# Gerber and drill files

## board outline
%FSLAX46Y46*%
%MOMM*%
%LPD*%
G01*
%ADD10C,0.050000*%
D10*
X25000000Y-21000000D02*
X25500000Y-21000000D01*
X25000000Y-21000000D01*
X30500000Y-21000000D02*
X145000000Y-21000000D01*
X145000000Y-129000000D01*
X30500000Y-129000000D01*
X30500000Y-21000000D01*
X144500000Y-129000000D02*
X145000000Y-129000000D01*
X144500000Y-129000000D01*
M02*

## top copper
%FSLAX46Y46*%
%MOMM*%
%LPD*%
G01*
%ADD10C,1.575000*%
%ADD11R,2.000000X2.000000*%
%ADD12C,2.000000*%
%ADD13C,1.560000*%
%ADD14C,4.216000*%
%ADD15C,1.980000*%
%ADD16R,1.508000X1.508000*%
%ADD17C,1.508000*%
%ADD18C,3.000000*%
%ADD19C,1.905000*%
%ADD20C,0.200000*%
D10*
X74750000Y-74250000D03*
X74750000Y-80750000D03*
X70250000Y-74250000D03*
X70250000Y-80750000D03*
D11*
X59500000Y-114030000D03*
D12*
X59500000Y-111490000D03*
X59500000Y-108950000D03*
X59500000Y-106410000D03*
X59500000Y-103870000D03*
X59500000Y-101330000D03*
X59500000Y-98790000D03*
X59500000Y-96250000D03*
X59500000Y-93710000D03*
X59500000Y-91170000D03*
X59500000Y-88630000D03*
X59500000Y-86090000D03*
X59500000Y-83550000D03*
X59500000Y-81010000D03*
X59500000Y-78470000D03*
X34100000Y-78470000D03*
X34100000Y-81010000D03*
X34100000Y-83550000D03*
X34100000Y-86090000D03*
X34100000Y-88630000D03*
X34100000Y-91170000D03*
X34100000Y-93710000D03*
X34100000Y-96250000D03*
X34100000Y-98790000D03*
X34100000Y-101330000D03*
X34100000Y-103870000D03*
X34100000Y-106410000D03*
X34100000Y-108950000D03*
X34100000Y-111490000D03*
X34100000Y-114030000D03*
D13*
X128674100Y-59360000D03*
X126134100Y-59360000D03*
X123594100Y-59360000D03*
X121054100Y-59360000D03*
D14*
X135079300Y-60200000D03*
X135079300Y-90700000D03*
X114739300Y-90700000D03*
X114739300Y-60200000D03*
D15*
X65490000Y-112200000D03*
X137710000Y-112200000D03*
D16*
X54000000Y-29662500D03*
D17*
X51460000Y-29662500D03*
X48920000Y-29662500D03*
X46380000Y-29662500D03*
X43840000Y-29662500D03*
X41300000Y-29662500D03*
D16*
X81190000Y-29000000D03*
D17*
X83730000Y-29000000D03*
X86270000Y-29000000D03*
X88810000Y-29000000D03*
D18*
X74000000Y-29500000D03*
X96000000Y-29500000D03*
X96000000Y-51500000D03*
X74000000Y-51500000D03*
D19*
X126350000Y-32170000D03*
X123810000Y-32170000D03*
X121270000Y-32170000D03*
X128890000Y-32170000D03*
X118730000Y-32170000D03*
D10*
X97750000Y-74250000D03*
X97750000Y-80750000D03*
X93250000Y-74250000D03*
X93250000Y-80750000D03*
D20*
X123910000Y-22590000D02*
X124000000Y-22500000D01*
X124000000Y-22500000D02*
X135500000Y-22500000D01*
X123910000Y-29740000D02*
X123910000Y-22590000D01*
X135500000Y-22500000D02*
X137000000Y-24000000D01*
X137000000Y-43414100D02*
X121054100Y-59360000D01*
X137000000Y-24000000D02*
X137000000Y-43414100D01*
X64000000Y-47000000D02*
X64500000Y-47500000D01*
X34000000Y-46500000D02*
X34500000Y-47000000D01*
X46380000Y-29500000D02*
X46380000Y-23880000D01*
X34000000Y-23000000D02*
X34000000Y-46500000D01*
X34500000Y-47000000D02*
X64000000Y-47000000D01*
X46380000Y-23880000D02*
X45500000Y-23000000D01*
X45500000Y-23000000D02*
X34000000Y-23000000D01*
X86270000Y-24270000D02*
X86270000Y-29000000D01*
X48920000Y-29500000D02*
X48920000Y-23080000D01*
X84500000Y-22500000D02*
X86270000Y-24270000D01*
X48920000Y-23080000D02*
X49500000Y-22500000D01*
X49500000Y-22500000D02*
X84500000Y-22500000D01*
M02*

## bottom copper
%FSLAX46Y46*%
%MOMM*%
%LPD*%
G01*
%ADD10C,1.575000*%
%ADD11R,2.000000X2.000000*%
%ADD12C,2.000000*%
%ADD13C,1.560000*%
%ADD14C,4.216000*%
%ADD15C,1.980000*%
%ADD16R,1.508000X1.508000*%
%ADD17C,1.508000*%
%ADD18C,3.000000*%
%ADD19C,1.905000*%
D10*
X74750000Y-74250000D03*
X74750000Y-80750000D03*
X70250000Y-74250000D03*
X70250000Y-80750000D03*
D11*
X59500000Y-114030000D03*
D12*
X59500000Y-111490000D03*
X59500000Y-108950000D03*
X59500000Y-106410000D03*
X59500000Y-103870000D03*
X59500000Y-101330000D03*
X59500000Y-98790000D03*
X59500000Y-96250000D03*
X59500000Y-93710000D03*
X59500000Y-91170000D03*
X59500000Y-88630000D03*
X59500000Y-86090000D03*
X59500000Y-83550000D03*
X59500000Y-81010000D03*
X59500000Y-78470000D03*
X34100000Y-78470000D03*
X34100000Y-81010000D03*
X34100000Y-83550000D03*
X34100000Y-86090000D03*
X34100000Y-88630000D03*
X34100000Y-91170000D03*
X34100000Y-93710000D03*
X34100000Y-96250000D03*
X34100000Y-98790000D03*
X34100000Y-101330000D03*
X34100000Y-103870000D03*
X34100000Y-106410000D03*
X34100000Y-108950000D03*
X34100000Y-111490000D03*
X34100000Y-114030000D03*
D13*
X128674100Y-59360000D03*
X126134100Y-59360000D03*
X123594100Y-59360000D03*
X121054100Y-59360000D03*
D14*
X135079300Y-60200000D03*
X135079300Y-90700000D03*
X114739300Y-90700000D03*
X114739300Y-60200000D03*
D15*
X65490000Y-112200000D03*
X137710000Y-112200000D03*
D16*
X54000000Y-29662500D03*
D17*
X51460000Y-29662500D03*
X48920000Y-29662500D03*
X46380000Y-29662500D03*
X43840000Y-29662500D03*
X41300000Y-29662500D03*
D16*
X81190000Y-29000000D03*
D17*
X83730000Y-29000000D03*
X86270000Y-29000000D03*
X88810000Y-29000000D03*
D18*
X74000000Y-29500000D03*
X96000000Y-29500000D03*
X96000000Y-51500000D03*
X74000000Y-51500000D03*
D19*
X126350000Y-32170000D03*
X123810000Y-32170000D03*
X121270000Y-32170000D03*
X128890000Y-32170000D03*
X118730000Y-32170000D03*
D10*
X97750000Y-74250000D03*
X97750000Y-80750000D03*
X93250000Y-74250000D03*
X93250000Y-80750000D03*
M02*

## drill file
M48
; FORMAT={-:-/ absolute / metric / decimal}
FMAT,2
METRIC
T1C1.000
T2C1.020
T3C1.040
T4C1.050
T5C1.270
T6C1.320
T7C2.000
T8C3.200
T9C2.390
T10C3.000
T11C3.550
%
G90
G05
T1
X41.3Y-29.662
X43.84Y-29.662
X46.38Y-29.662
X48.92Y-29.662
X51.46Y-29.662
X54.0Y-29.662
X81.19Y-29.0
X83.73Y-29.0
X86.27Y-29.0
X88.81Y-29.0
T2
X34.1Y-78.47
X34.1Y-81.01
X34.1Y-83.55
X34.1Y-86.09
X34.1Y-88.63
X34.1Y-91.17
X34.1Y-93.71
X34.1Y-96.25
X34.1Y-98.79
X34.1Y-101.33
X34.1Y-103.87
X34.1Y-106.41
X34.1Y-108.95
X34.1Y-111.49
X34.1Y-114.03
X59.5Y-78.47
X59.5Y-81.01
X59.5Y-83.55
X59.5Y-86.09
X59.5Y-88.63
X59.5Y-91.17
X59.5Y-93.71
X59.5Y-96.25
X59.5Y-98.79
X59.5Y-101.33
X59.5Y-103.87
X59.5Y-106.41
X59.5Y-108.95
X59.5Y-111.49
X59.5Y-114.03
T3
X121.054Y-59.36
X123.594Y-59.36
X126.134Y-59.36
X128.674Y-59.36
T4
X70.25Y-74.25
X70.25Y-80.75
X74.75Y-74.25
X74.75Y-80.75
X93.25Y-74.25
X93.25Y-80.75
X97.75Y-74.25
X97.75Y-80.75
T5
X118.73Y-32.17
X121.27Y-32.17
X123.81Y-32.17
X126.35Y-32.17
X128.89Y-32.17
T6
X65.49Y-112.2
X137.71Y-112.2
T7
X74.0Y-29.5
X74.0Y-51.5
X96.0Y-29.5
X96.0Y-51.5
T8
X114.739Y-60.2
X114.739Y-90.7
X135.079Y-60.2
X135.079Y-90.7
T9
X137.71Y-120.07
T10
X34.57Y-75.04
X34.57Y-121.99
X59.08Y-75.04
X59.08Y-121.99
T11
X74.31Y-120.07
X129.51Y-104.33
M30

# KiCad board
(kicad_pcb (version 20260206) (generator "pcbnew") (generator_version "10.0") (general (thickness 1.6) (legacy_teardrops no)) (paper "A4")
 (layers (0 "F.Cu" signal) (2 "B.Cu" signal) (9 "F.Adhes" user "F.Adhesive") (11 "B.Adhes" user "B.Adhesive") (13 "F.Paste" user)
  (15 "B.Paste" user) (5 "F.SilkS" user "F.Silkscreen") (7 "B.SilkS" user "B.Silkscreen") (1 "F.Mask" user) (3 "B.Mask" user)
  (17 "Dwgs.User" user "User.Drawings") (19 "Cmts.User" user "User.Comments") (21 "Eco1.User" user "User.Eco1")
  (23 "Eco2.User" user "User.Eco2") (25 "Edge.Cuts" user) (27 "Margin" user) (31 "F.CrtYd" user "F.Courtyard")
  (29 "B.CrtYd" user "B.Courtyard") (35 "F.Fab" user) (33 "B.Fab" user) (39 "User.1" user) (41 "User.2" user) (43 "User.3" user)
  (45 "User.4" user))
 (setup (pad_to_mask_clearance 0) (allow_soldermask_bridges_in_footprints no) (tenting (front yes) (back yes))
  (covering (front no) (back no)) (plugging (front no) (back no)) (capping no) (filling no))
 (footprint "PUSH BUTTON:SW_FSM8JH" (layer "F.Cu") (at 72.5 77.5)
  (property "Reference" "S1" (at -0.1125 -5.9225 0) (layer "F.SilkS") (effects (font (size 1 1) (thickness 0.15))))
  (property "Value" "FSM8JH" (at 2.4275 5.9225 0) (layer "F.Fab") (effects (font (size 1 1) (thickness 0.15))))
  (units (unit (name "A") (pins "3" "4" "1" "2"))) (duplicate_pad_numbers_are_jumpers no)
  (pad "1" thru_hole circle (at 2.25 -3.25) (size 1.575 1.575) (drill 1.05) (layers "*.Cu" "*.Mask") (remove_unused_layers no)
   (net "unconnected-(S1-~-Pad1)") (solder_mask_margin 0.102))
  (pad "2" thru_hole circle (at 2.25 3.25) (size 1.575 1.575) (drill 1.05) (layers "*.Cu" "*.Mask") (remove_unused_layers no)
   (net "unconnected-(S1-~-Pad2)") (solder_mask_margin 0.102))
  (pad "3" thru_hole circle (at -2.25 -3.25) (size 1.575 1.575) (drill 1.05) (layers "*.Cu" "*.Mask") (remove_unused_layers no)
   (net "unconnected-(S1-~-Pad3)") (solder_mask_margin 0.102))
  (pad "4" thru_hole circle (at -2.25 3.25) (size 1.575 1.575) (drill 1.05) (layers "*.Cu" "*.Mask") (remove_unused_layers no)
   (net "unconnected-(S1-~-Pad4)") (solder_mask_margin 0.102)))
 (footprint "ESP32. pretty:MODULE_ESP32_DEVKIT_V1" (layer "F.Cu") (at 46.8 98.515 180)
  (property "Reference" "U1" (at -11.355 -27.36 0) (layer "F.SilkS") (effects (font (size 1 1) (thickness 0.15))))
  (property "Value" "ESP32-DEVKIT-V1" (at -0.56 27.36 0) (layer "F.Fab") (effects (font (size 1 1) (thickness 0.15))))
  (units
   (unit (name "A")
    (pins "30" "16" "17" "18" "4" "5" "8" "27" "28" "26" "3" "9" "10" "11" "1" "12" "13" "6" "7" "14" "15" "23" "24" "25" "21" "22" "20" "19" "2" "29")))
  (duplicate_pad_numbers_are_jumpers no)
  (pad "" np_thru_hole circle (at -12.28 -23.475 180) (size 3 3) (drill 3) (layers "*.Cu" "*.Mask"))
  (pad "" np_thru_hole circle (at -12.28 23.475 180) (size 3 3) (drill 3) (layers "*.Cu" "*.Mask"))
  (pad "" np_thru_hole circle (at 12.23 -23.475 180) (size 3 3) (drill 3) (layers "*.Cu" "*.Mask"))
  (pad "" np_thru_hole circle (at 12.23 23.475 180) (size 3 3) (drill 3) (layers "*.Cu" "*.Mask"))
  (pad "1" thru_hole rect (at -12.7 -15.515 180) (size 2 2) (drill 1.02) (layers "*.Cu" "*.Mask") (remove_unused_layers no)
   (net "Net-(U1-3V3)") (solder_mask_margin 0.102))
  (pad "2" thru_hole circle (at -12.7 -12.975 180) (size 2 2) (drill 1.02) (layers "*.Cu" "*.Mask") (remove_unused_layers no)
   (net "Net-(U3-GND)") (solder_mask_margin 0.102))
  (pad "3" thru_hole circle (at -12.7 -10.435 180) (size 2 2) (drill 1.02) (layers "*.Cu" "*.Mask") (remove_unused_layers no)
   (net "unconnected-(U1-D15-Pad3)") (solder_mask_margin 0.102))
  (pad "4" thru_hole circle (at -12.7 -7.895 180) (size 2 2) (drill 1.02) (layers "*.Cu" "*.Mask") (remove_unused_layers no)
   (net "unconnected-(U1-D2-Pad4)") (solder_mask_margin 0.102))
  (pad "5" thru_hole circle (at -12.7 -5.355 180) (size 2 2) (drill 1.02) (layers "*.Cu" "*.Mask") (remove_unused_layers no)
   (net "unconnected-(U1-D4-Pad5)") (solder_mask_margin 0.102))
  (pad "6" thru_hole circle (at -12.7 -2.815 180) (size 2 2) (drill 1.02) (layers "*.Cu" "*.Mask") (remove_unused_layers no)
   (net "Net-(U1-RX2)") (solder_mask_margin 0.102))
  (pad "7" thru_hole circle (at -12.7 -0.275 180) (size 2 2) (drill 1.02) (layers "*.Cu" "*.Mask") (remove_unused_layers no)
   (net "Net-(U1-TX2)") (solder_mask_margin 0.102))
  (pad "8" thru_hole circle (at -12.7 2.265 180) (size 2 2) (drill 1.02) (layers "*.Cu" "*.Mask") (remove_unused_layers no)
   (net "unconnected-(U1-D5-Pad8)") (solder_mask_margin 0.102))
  (pad "9" thru_hole circle (at -12.7 4.805 180) (size 2 2) (drill 1.02) (layers "*.Cu" "*.Mask") (remove_unused_layers no)
   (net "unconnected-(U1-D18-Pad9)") (solder_mask_margin 0.102))
  (pad "10" thru_hole circle (at -12.7 7.345 180) (size 2 2) (drill 1.02) (layers "*.Cu" "*.Mask") (remove_unused_layers no)
   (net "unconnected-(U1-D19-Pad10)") (solder_mask_margin 0.102))
  (pad "11" thru_hole circle (at -12.7 9.885 180) (size 2 2) (drill 1.02) (layers "*.Cu" "*.Mask") (remove_unused_layers no)
   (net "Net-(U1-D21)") (solder_mask_margin 0.102))
  (pad "12" thru_hole circle (at -12.7 12.425 180) (size 2 2) (drill 1.02) (layers "*.Cu" "*.Mask") (remove_unused_layers no)
   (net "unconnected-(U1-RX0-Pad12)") (solder_mask_margin 0.102))
  (pad "13" thru_hole circle (at -12.7 14.965 180) (size 2 2) (drill 1.02) (layers "*.Cu" "*.Mask") (remove_unused_layers no)
   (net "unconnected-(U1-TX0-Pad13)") (solder_mask_margin 0.102))
  (pad "14" thru_hole circle (at -12.7 17.505 180) (size 2 2) (drill 1.02) (layers "*.Cu" "*.Mask") (remove_unused_layers no)
   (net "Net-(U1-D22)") (solder_mask_margin 0.102))
  (pad "15" thru_hole circle (at -12.7 20.045 180) (size 2 2) (drill 1.02) (layers "*.Cu" "*.Mask") (remove_unused_layers no)
   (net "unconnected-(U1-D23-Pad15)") (solder_mask_margin 0.102))
  (pad "16" thru_hole circle (at 12.7 20.045 180) (size 2 2) (drill 1.02) (layers "*.Cu" "*.Mask") (remove_unused_layers no)
   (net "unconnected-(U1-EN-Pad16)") (solder_mask_margin 0.102))
  (pad "17" thru_hole circle (at 12.7 17.505 180) (size 2 2) (drill 1.02) (layers "*.Cu" "*.Mask") (remove_unused_layers no)
   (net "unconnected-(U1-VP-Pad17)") (solder_mask_margin 0.102))
  (pad "18" thru_hole circle (at 12.7 14.965 180) (size 2 2) (drill 1.02) (layers "*.Cu" "*.Mask") (remove_unused_layers no)
   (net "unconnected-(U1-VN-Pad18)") (solder_mask_margin 0.102))
  (pad "19" thru_hole circle (at 12.7 12.425 180) (size 2 2) (drill 1.02) (layers "*.Cu" "*.Mask") (remove_unused_layers no)
   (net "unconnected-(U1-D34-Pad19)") (solder_mask_margin 0.102))
  (pad "20" thru_hole circle (at 12.7 9.885 180) (size 2 2) (drill 1.02) (layers "*.Cu" "*.Mask") (remove_unused_layers no)
   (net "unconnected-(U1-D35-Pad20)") (solder_mask_margin 0.102))
  (pad "21" thru_hole circle (at 12.7 7.345 180) (size 2 2) (drill 1.02) (layers "*.Cu" "*.Mask") (remove_unused_layers no)
   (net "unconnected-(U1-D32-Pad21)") (solder_mask_margin 0.102))
  (pad "22" thru_hole circle (at 12.7 4.805 180) (size 2 2) (drill 1.02) (layers "*.Cu" "*.Mask") (remove_unused_layers no)
   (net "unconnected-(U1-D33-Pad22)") (solder_mask_margin 0.102))
  (pad "23" thru_hole circle (at 12.7 2.265 180) (size 2 2) (drill 1.02) (layers "*.Cu" "*.Mask") (remove_unused_layers no)
   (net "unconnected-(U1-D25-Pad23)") (solder_mask_margin 0.102))
  (pad "24" thru_hole circle (at 12.7 -0.275 180) (size 2 2) (drill 1.02) (layers "*.Cu" "*.Mask") (remove_unused_layers no)
   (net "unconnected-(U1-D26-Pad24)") (solder_mask_margin 0.102))
  (pad "25" thru_hole circle (at 12.7 -2.815 180) (size 2 2) (drill 1.02) (layers "*.Cu" "*.Mask") (remove_unused_layers no)
   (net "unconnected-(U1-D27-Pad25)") (solder_mask_margin 0.102))
  (pad "26" thru_hole circle (at 12.7 -5.355 180) (size 2 2) (drill 1.02) (layers "*.Cu" "*.Mask") (remove_unused_layers no)
   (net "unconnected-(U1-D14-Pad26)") (solder_mask_margin 0.102))
  (pad "27" thru_hole circle (at 12.7 -7.895 180) (size 2 2) (drill 1.02) (layers "*.Cu" "*.Mask") (remove_unused_layers no)
   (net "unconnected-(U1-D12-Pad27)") (solder_mask_margin 0.102))
  (pad "28" thru_hole circle (at 12.7 -10.435 180) (size 2 2) (drill 1.02) (layers "*.Cu" "*.Mask") (remove_unused_layers no)
   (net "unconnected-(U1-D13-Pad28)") (solder_mask_margin 0.102))
  (pad "29" thru_hole circle (at 12.7 -12.975 180) (size 2 2) (drill 1.02) (layers "*.Cu" "*.Mask") (remove_unused_layers no)
   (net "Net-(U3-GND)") (solder_mask_margin 0.102))
  (pad "30" thru_hole circle (at 12.7 -15.515 180) (size 2 2) (drill 1.02) (layers "*.Cu" "*.Mask") (remove_unused_layers no)
   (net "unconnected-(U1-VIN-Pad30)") (solder_mask_margin 0.102)))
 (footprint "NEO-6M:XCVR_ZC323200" (layer "F.Cu") (at 124.5 75.5 180)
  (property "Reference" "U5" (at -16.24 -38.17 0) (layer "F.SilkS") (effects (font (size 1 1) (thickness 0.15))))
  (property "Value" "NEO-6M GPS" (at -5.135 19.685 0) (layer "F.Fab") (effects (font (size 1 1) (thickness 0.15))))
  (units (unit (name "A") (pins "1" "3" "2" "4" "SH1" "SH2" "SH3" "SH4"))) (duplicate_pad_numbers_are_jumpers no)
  (pad "1" thru_hole circle (at -4.1741 16.14 180) (size 1.56 1.56) (drill 1.04) (layers "*.Cu" "*.Mask") (remove_unused_layers no)
   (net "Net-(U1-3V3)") (solder_mask_margin 0.102))
  (pad "2" thru_hole circle (at -1.6341 16.14 180) (size 1.56 1.56) (drill 1.04) (layers "*.Cu" "*.Mask") (remove_unused_layers no)
   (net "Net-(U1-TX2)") (solder_mask_margin 0.102))
  (pad "3" thru_hole circle (at 0.9059 16.14 180) (size 1.56 1.56) (drill 1.04) (layers "*.Cu" "*.Mask") (remove_unused_layers no)
   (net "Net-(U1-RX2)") (solder_mask_margin 0.102))
  (pad "4" thru_hole circle (at 3.4459 16.14 180) (size 1.56 1.56) (drill 1.04) (layers "*.Cu" "*.Mask") (remove_unused_layers no)
   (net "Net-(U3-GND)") (solder_mask_margin 0.102))
  (pad "SH1" thru_hole circle (at -10.5793 15.3 180) (size 4.216 4.216) (drill 3.2) (layers "*.Cu" "*.Mask") (remove_unused_layers no)
   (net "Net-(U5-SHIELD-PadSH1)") (solder_mask_margin 0.102))
  (pad "SH2" thru_hole circle (at -10.5793 -15.2 180) (size 4.216 4.216) (drill 3.2) (layers "*.Cu" "*.Mask") (remove_unused_layers no)
   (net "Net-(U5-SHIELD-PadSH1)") (solder_mask_margin 0.102))
  (pad "SH3" thru_hole circle (at 9.7607 -15.2 180) (size 4.216 4.216) (drill 3.2) (layers "*.Cu" "*.Mask") (remove_unused_layers no)
   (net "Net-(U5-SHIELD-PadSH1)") (solder_mask_margin 0.102))
  (pad "SH4" thru_hole circle (at 9.7607 15.3 180) (size 4.216 4.216) (drill 3.2) (layers "*.Cu" "*.Mask") (remove_unused_layers no)
   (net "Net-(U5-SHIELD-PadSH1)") (solder_mask_margin 0.102)))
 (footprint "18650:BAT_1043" (layer "F.Cu") (at 101.6 112.2)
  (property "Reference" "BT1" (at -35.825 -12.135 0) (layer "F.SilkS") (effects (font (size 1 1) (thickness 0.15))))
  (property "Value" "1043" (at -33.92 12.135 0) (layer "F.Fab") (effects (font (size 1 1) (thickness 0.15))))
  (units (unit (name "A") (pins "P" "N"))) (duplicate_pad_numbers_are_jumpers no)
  (pad "" np_thru_hole circle (at -27.29 7.87) (size 3.55 3.55) (drill 3.55) (layers "*.Cu" "*.Mask"))
  (pad "" np_thru_hole circle (at 27.91 -7.87) (size 3.55 3.55) (drill 3.55) (layers "*.Cu" "*.Mask"))
  (pad "" np_thru_hole circle (at 36.11 7.87) (size 2.39 2.39) (drill 2.39) (layers "*.Cu" "*.Mask"))
  (pad "N" thru_hole circle (at -36.11 0) (size 1.98 1.98) (drill 1.32) (layers "*.Cu" "*.Mask") (remove_unused_layers no)
   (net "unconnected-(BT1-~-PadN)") (solder_mask_margin 0.102))
  (pad "P" thru_hole circle (at 36.11 0) (size 1.98 1.98) (drill 1.32) (layers "*.Cu" "*.Mask") (remove_unused_layers no)
   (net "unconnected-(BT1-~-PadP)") (solder_mask_margin 0.102)))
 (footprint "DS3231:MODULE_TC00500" (layer "F.Cu") (at 47.65 29.6625 -90)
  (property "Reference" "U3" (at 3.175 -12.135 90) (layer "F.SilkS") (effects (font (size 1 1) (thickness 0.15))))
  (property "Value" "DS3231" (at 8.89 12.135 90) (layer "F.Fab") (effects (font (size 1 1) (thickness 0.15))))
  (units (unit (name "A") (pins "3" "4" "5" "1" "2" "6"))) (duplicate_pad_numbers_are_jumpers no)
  (pad "1" thru_hole rect (at 0 -6.35 270) (size 1.508 1.508) (drill 1) (layers "*.Cu" "*.Mask") (remove_unused_layers no)
   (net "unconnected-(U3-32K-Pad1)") (solder_mask_margin 0.102))
  (pad "2" thru_hole circle (at 0 -3.81 270) (size 1.508 1.508) (drill 1) (layers "*.Cu" "*.Mask") (remove_unused_layers no)
   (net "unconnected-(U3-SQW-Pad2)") (solder_mask_margin 0.102))
  (pad "3" thru_hole circle (at 0 -1.27 270) (size 1.508 1.508) (drill 1) (layers "*.Cu" "*.Mask") (remove_unused_layers no)
   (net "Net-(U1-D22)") (solder_mask_margin 0.102))
  (pad "4" thru_hole circle (at 0 1.27 270) (size 1.508 1.508) (drill 1) (layers "*.Cu" "*.Mask") (remove_unused_layers no)
   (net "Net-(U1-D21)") (solder_mask_margin 0.102))
  (pad "5" thru_hole circle (at 0 3.81 270) (size 1.508 1.508) (drill 1) (layers "*.Cu" "*.Mask") (remove_unused_layers no)
   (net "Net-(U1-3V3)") (solder_mask_margin 0.102))
  (pad "6" thru_hole circle (at 0 6.35 270) (size 1.508 1.508) (drill 1) (layers "*.Cu" "*.Mask") (remove_unused_layers no)
   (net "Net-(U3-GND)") (solder_mask_margin 0.102)))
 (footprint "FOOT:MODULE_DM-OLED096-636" (layer "F.Cu") (at 85 40.5)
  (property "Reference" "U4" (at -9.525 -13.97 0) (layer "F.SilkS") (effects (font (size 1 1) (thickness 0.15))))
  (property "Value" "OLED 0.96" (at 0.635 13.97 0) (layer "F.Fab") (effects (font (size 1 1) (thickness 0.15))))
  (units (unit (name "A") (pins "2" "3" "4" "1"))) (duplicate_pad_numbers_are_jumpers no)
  (pad "1" thru_hole rect (at -3.81 -11.5) (size 1.508 1.508) (drill 1) (layers "*.Cu" "*.Mask") (remove_unused_layers no)
   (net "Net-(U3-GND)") (solder_mask_margin 0.102))
  (pad "2" thru_hole circle (at -1.27 -11.5) (size 1.508 1.508) (drill 1) (layers "*.Cu" "*.Mask") (remove_unused_layers no)
   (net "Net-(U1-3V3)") (solder_mask_margin 0.102))
  (pad "3" thru_hole circle (at 1.27 -11.5) (size 1.508 1.508) (drill 1) (layers "*.Cu" "*.Mask") (remove_unused_layers no)
   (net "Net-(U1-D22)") (solder_mask_margin 0.102))
  (pad "4" thru_hole circle (at 3.81 -11.5) (size 1.508 1.508) (drill 1) (layers "*.Cu" "*.Mask") (remove_unused_layers no)
   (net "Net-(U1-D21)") (solder_mask_margin 0.102))
  (pad "S1" thru_hole circle (at -11 -11) (size 3 3) (drill 2) (layers "*.Cu" "*.Mask") (remove_unused_layers no) (solder_mask_margin 0.102))
  (pad "S2" thru_hole circle (at 11 -11) (size 3 3) (drill 2) (layers "*.Cu" "*.Mask") (remove_unused_layers no) (solder_mask_margin 0.102))
  (pad "S3" thru_hole circle (at 11 11) (size 3 3) (drill 2) (layers "*.Cu" "*.Mask") (remove_unused_layers no) (solder_mask_margin 0.102))
  (pad "S4" thru_hole circle (at -11 11) (size 3 3) (drill 2) (layers "*.Cu" "*.Mask") (remove_unused_layers no) (solder_mask_margin 0.102)))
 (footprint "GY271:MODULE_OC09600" (layer "F.Cu") (at 120 38.5 -90)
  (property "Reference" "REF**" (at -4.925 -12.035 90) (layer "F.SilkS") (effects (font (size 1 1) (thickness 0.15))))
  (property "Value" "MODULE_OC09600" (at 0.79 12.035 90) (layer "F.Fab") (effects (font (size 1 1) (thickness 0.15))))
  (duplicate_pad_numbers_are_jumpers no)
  (pad "GND" thru_hole circle (at -6.33 -6.35 270) (size 1.905 1.905) (drill 1.27) (layers "*.Cu" "*.Mask") (remove_unused_layers no)
   (solder_mask_margin 0.102))
  (pad "SCL" thru_hole circle (at -6.33 -3.81 270) (size 1.905 1.905) (drill 1.27) (layers "*.Cu" "*.Mask") (remove_unused_layers no)
   (solder_mask_margin 0.102))
  (pad "SDA" thru_hole circle (at -6.33 -1.27 270) (size 1.905 1.905) (drill 1.27) (layers "*.Cu" "*.Mask") (remove_unused_layers no)
   (solder_mask_margin 0.102))
  (pad "VCC" thru_hole circle (at -6.33 -8.89 270) (size 1.905 1.905) (drill 1.27) (layers "*.Cu" "*.Mask") (remove_unused_layers no)
   (solder_mask_margin 0.102))
  (pad "XDA" thru_hole circle (at -6.33 1.27 270) (size 1.905 1.905) (drill 1.27) (layers "*.Cu" "*.Mask") (remove_unused_layers no)
   (solder_mask_margin 0.102)))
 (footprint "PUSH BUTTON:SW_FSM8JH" (layer "F.Cu") (at 95.5 77.5)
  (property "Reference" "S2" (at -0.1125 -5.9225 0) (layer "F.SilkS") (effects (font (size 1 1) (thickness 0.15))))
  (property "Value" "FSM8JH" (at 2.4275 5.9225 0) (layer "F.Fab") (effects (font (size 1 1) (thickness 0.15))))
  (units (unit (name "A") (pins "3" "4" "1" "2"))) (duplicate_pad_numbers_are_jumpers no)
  (pad "1" thru_hole circle (at 2.25 -3.25) (size 1.575 1.575) (drill 1.05) (layers "*.Cu" "*.Mask") (remove_unused_layers no)
   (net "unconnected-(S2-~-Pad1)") (solder_mask_margin 0.102))
  (pad "2" thru_hole circle (at 2.25 3.25) (size 1.575 1.575) (drill 1.05) (layers "*.Cu" "*.Mask") (remove_unused_layers no)
   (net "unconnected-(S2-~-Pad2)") (solder_mask_margin 0.102))
  (pad "3" thru_hole circle (at -2.25 -3.25) (size 1.575 1.575) (drill 1.05) (layers "*.Cu" "*.Mask") (remove_unused_layers no)
   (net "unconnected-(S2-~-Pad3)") (solder_mask_margin 0.102))
  (pad "4" thru_hole circle (at -2.25 3.25) (size 1.575 1.575) (drill 1.05) (layers "*.Cu" "*.Mask") (remove_unused_layers no)
   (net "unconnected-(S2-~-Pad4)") (solder_mask_margin 0.102)))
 (gr_rect (start 25 21) (end 25.5 21) (stroke (width 0.05) (type default)) (fill no) (layer "Edge.Cuts"))
 (gr_rect (start 30.5 21) (end 145 129) (stroke (width 0.05) (type default)) (fill no) (layer "Edge.Cuts"))
 (gr_rect (start 144.5 129) (end 145 129) (stroke (width 0.05) (type default)) (fill no) (layer "Edge.Cuts"))
 (segment (start 123.91 22.59) (end 124 22.5) (width 0.2) (layer "F.Cu") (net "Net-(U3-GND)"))
 (segment (start 124 22.5) (end 135.5 22.5) (width 0.2) (layer "F.Cu") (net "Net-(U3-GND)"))
 (segment (start 123.91 29.74) (end 123.91 22.59) (width 0.2) (layer "F.Cu") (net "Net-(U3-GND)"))
 (segment (start 135.5 22.5) (end 137 24) (width 0.2) (layer "F.Cu") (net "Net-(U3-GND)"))
 (segment (start 137 43.4141) (end 121.0541 59.36) (width 0.2) (layer "F.Cu") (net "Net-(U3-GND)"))
 (segment (start 137 24) (end 137 43.4141) (width 0.2) (layer "F.Cu") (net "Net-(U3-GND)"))
 (segment (start 64 47) (end 64.5 47.5) (width 0.2) (layer "F.Cu") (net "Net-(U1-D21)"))
 (segment (start 34 46.5) (end 34.5 47) (width 0.2) (layer "F.Cu") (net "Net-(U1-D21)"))
 (segment (start 46.38 29.5) (end 46.38 23.88) (width 0.2) (layer "F.Cu") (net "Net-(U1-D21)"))
 (segment (start 34 23) (end 34 46.5) (width 0.2) (layer "F.Cu") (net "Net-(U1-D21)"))
 (segment (start 34.5 47) (end 64 47) (width 0.2) (layer "F.Cu") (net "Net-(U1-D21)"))
 (segment (start 46.38 23.88) (end 45.5 23) (width 0.2) (layer "F.Cu") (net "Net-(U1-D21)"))
 (segment (start 45.5 23) (end 34 23) (width 0.2) (layer "F.Cu") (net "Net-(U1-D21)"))
 (segment (start 86.27 24.27) (end 86.27 29) (width 0.2) (layer "F.Cu") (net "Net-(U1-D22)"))
 (segment (start 48.92 29.5) (end 48.92 23.08) (width 0.2) (layer "F.Cu") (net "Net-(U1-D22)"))
 (segment (start 84.5 22.5) (end 86.27 24.27) (width 0.2) (layer "F.Cu") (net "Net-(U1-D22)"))
 (segment (start 48.92 23.08) (end 49.5 22.5) (width 0.2) (layer "F.Cu") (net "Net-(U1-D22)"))
 (segment (start 49.5 22.5) (end 84.5 22.5) (width 0.2) (layer "F.Cu") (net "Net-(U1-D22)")))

